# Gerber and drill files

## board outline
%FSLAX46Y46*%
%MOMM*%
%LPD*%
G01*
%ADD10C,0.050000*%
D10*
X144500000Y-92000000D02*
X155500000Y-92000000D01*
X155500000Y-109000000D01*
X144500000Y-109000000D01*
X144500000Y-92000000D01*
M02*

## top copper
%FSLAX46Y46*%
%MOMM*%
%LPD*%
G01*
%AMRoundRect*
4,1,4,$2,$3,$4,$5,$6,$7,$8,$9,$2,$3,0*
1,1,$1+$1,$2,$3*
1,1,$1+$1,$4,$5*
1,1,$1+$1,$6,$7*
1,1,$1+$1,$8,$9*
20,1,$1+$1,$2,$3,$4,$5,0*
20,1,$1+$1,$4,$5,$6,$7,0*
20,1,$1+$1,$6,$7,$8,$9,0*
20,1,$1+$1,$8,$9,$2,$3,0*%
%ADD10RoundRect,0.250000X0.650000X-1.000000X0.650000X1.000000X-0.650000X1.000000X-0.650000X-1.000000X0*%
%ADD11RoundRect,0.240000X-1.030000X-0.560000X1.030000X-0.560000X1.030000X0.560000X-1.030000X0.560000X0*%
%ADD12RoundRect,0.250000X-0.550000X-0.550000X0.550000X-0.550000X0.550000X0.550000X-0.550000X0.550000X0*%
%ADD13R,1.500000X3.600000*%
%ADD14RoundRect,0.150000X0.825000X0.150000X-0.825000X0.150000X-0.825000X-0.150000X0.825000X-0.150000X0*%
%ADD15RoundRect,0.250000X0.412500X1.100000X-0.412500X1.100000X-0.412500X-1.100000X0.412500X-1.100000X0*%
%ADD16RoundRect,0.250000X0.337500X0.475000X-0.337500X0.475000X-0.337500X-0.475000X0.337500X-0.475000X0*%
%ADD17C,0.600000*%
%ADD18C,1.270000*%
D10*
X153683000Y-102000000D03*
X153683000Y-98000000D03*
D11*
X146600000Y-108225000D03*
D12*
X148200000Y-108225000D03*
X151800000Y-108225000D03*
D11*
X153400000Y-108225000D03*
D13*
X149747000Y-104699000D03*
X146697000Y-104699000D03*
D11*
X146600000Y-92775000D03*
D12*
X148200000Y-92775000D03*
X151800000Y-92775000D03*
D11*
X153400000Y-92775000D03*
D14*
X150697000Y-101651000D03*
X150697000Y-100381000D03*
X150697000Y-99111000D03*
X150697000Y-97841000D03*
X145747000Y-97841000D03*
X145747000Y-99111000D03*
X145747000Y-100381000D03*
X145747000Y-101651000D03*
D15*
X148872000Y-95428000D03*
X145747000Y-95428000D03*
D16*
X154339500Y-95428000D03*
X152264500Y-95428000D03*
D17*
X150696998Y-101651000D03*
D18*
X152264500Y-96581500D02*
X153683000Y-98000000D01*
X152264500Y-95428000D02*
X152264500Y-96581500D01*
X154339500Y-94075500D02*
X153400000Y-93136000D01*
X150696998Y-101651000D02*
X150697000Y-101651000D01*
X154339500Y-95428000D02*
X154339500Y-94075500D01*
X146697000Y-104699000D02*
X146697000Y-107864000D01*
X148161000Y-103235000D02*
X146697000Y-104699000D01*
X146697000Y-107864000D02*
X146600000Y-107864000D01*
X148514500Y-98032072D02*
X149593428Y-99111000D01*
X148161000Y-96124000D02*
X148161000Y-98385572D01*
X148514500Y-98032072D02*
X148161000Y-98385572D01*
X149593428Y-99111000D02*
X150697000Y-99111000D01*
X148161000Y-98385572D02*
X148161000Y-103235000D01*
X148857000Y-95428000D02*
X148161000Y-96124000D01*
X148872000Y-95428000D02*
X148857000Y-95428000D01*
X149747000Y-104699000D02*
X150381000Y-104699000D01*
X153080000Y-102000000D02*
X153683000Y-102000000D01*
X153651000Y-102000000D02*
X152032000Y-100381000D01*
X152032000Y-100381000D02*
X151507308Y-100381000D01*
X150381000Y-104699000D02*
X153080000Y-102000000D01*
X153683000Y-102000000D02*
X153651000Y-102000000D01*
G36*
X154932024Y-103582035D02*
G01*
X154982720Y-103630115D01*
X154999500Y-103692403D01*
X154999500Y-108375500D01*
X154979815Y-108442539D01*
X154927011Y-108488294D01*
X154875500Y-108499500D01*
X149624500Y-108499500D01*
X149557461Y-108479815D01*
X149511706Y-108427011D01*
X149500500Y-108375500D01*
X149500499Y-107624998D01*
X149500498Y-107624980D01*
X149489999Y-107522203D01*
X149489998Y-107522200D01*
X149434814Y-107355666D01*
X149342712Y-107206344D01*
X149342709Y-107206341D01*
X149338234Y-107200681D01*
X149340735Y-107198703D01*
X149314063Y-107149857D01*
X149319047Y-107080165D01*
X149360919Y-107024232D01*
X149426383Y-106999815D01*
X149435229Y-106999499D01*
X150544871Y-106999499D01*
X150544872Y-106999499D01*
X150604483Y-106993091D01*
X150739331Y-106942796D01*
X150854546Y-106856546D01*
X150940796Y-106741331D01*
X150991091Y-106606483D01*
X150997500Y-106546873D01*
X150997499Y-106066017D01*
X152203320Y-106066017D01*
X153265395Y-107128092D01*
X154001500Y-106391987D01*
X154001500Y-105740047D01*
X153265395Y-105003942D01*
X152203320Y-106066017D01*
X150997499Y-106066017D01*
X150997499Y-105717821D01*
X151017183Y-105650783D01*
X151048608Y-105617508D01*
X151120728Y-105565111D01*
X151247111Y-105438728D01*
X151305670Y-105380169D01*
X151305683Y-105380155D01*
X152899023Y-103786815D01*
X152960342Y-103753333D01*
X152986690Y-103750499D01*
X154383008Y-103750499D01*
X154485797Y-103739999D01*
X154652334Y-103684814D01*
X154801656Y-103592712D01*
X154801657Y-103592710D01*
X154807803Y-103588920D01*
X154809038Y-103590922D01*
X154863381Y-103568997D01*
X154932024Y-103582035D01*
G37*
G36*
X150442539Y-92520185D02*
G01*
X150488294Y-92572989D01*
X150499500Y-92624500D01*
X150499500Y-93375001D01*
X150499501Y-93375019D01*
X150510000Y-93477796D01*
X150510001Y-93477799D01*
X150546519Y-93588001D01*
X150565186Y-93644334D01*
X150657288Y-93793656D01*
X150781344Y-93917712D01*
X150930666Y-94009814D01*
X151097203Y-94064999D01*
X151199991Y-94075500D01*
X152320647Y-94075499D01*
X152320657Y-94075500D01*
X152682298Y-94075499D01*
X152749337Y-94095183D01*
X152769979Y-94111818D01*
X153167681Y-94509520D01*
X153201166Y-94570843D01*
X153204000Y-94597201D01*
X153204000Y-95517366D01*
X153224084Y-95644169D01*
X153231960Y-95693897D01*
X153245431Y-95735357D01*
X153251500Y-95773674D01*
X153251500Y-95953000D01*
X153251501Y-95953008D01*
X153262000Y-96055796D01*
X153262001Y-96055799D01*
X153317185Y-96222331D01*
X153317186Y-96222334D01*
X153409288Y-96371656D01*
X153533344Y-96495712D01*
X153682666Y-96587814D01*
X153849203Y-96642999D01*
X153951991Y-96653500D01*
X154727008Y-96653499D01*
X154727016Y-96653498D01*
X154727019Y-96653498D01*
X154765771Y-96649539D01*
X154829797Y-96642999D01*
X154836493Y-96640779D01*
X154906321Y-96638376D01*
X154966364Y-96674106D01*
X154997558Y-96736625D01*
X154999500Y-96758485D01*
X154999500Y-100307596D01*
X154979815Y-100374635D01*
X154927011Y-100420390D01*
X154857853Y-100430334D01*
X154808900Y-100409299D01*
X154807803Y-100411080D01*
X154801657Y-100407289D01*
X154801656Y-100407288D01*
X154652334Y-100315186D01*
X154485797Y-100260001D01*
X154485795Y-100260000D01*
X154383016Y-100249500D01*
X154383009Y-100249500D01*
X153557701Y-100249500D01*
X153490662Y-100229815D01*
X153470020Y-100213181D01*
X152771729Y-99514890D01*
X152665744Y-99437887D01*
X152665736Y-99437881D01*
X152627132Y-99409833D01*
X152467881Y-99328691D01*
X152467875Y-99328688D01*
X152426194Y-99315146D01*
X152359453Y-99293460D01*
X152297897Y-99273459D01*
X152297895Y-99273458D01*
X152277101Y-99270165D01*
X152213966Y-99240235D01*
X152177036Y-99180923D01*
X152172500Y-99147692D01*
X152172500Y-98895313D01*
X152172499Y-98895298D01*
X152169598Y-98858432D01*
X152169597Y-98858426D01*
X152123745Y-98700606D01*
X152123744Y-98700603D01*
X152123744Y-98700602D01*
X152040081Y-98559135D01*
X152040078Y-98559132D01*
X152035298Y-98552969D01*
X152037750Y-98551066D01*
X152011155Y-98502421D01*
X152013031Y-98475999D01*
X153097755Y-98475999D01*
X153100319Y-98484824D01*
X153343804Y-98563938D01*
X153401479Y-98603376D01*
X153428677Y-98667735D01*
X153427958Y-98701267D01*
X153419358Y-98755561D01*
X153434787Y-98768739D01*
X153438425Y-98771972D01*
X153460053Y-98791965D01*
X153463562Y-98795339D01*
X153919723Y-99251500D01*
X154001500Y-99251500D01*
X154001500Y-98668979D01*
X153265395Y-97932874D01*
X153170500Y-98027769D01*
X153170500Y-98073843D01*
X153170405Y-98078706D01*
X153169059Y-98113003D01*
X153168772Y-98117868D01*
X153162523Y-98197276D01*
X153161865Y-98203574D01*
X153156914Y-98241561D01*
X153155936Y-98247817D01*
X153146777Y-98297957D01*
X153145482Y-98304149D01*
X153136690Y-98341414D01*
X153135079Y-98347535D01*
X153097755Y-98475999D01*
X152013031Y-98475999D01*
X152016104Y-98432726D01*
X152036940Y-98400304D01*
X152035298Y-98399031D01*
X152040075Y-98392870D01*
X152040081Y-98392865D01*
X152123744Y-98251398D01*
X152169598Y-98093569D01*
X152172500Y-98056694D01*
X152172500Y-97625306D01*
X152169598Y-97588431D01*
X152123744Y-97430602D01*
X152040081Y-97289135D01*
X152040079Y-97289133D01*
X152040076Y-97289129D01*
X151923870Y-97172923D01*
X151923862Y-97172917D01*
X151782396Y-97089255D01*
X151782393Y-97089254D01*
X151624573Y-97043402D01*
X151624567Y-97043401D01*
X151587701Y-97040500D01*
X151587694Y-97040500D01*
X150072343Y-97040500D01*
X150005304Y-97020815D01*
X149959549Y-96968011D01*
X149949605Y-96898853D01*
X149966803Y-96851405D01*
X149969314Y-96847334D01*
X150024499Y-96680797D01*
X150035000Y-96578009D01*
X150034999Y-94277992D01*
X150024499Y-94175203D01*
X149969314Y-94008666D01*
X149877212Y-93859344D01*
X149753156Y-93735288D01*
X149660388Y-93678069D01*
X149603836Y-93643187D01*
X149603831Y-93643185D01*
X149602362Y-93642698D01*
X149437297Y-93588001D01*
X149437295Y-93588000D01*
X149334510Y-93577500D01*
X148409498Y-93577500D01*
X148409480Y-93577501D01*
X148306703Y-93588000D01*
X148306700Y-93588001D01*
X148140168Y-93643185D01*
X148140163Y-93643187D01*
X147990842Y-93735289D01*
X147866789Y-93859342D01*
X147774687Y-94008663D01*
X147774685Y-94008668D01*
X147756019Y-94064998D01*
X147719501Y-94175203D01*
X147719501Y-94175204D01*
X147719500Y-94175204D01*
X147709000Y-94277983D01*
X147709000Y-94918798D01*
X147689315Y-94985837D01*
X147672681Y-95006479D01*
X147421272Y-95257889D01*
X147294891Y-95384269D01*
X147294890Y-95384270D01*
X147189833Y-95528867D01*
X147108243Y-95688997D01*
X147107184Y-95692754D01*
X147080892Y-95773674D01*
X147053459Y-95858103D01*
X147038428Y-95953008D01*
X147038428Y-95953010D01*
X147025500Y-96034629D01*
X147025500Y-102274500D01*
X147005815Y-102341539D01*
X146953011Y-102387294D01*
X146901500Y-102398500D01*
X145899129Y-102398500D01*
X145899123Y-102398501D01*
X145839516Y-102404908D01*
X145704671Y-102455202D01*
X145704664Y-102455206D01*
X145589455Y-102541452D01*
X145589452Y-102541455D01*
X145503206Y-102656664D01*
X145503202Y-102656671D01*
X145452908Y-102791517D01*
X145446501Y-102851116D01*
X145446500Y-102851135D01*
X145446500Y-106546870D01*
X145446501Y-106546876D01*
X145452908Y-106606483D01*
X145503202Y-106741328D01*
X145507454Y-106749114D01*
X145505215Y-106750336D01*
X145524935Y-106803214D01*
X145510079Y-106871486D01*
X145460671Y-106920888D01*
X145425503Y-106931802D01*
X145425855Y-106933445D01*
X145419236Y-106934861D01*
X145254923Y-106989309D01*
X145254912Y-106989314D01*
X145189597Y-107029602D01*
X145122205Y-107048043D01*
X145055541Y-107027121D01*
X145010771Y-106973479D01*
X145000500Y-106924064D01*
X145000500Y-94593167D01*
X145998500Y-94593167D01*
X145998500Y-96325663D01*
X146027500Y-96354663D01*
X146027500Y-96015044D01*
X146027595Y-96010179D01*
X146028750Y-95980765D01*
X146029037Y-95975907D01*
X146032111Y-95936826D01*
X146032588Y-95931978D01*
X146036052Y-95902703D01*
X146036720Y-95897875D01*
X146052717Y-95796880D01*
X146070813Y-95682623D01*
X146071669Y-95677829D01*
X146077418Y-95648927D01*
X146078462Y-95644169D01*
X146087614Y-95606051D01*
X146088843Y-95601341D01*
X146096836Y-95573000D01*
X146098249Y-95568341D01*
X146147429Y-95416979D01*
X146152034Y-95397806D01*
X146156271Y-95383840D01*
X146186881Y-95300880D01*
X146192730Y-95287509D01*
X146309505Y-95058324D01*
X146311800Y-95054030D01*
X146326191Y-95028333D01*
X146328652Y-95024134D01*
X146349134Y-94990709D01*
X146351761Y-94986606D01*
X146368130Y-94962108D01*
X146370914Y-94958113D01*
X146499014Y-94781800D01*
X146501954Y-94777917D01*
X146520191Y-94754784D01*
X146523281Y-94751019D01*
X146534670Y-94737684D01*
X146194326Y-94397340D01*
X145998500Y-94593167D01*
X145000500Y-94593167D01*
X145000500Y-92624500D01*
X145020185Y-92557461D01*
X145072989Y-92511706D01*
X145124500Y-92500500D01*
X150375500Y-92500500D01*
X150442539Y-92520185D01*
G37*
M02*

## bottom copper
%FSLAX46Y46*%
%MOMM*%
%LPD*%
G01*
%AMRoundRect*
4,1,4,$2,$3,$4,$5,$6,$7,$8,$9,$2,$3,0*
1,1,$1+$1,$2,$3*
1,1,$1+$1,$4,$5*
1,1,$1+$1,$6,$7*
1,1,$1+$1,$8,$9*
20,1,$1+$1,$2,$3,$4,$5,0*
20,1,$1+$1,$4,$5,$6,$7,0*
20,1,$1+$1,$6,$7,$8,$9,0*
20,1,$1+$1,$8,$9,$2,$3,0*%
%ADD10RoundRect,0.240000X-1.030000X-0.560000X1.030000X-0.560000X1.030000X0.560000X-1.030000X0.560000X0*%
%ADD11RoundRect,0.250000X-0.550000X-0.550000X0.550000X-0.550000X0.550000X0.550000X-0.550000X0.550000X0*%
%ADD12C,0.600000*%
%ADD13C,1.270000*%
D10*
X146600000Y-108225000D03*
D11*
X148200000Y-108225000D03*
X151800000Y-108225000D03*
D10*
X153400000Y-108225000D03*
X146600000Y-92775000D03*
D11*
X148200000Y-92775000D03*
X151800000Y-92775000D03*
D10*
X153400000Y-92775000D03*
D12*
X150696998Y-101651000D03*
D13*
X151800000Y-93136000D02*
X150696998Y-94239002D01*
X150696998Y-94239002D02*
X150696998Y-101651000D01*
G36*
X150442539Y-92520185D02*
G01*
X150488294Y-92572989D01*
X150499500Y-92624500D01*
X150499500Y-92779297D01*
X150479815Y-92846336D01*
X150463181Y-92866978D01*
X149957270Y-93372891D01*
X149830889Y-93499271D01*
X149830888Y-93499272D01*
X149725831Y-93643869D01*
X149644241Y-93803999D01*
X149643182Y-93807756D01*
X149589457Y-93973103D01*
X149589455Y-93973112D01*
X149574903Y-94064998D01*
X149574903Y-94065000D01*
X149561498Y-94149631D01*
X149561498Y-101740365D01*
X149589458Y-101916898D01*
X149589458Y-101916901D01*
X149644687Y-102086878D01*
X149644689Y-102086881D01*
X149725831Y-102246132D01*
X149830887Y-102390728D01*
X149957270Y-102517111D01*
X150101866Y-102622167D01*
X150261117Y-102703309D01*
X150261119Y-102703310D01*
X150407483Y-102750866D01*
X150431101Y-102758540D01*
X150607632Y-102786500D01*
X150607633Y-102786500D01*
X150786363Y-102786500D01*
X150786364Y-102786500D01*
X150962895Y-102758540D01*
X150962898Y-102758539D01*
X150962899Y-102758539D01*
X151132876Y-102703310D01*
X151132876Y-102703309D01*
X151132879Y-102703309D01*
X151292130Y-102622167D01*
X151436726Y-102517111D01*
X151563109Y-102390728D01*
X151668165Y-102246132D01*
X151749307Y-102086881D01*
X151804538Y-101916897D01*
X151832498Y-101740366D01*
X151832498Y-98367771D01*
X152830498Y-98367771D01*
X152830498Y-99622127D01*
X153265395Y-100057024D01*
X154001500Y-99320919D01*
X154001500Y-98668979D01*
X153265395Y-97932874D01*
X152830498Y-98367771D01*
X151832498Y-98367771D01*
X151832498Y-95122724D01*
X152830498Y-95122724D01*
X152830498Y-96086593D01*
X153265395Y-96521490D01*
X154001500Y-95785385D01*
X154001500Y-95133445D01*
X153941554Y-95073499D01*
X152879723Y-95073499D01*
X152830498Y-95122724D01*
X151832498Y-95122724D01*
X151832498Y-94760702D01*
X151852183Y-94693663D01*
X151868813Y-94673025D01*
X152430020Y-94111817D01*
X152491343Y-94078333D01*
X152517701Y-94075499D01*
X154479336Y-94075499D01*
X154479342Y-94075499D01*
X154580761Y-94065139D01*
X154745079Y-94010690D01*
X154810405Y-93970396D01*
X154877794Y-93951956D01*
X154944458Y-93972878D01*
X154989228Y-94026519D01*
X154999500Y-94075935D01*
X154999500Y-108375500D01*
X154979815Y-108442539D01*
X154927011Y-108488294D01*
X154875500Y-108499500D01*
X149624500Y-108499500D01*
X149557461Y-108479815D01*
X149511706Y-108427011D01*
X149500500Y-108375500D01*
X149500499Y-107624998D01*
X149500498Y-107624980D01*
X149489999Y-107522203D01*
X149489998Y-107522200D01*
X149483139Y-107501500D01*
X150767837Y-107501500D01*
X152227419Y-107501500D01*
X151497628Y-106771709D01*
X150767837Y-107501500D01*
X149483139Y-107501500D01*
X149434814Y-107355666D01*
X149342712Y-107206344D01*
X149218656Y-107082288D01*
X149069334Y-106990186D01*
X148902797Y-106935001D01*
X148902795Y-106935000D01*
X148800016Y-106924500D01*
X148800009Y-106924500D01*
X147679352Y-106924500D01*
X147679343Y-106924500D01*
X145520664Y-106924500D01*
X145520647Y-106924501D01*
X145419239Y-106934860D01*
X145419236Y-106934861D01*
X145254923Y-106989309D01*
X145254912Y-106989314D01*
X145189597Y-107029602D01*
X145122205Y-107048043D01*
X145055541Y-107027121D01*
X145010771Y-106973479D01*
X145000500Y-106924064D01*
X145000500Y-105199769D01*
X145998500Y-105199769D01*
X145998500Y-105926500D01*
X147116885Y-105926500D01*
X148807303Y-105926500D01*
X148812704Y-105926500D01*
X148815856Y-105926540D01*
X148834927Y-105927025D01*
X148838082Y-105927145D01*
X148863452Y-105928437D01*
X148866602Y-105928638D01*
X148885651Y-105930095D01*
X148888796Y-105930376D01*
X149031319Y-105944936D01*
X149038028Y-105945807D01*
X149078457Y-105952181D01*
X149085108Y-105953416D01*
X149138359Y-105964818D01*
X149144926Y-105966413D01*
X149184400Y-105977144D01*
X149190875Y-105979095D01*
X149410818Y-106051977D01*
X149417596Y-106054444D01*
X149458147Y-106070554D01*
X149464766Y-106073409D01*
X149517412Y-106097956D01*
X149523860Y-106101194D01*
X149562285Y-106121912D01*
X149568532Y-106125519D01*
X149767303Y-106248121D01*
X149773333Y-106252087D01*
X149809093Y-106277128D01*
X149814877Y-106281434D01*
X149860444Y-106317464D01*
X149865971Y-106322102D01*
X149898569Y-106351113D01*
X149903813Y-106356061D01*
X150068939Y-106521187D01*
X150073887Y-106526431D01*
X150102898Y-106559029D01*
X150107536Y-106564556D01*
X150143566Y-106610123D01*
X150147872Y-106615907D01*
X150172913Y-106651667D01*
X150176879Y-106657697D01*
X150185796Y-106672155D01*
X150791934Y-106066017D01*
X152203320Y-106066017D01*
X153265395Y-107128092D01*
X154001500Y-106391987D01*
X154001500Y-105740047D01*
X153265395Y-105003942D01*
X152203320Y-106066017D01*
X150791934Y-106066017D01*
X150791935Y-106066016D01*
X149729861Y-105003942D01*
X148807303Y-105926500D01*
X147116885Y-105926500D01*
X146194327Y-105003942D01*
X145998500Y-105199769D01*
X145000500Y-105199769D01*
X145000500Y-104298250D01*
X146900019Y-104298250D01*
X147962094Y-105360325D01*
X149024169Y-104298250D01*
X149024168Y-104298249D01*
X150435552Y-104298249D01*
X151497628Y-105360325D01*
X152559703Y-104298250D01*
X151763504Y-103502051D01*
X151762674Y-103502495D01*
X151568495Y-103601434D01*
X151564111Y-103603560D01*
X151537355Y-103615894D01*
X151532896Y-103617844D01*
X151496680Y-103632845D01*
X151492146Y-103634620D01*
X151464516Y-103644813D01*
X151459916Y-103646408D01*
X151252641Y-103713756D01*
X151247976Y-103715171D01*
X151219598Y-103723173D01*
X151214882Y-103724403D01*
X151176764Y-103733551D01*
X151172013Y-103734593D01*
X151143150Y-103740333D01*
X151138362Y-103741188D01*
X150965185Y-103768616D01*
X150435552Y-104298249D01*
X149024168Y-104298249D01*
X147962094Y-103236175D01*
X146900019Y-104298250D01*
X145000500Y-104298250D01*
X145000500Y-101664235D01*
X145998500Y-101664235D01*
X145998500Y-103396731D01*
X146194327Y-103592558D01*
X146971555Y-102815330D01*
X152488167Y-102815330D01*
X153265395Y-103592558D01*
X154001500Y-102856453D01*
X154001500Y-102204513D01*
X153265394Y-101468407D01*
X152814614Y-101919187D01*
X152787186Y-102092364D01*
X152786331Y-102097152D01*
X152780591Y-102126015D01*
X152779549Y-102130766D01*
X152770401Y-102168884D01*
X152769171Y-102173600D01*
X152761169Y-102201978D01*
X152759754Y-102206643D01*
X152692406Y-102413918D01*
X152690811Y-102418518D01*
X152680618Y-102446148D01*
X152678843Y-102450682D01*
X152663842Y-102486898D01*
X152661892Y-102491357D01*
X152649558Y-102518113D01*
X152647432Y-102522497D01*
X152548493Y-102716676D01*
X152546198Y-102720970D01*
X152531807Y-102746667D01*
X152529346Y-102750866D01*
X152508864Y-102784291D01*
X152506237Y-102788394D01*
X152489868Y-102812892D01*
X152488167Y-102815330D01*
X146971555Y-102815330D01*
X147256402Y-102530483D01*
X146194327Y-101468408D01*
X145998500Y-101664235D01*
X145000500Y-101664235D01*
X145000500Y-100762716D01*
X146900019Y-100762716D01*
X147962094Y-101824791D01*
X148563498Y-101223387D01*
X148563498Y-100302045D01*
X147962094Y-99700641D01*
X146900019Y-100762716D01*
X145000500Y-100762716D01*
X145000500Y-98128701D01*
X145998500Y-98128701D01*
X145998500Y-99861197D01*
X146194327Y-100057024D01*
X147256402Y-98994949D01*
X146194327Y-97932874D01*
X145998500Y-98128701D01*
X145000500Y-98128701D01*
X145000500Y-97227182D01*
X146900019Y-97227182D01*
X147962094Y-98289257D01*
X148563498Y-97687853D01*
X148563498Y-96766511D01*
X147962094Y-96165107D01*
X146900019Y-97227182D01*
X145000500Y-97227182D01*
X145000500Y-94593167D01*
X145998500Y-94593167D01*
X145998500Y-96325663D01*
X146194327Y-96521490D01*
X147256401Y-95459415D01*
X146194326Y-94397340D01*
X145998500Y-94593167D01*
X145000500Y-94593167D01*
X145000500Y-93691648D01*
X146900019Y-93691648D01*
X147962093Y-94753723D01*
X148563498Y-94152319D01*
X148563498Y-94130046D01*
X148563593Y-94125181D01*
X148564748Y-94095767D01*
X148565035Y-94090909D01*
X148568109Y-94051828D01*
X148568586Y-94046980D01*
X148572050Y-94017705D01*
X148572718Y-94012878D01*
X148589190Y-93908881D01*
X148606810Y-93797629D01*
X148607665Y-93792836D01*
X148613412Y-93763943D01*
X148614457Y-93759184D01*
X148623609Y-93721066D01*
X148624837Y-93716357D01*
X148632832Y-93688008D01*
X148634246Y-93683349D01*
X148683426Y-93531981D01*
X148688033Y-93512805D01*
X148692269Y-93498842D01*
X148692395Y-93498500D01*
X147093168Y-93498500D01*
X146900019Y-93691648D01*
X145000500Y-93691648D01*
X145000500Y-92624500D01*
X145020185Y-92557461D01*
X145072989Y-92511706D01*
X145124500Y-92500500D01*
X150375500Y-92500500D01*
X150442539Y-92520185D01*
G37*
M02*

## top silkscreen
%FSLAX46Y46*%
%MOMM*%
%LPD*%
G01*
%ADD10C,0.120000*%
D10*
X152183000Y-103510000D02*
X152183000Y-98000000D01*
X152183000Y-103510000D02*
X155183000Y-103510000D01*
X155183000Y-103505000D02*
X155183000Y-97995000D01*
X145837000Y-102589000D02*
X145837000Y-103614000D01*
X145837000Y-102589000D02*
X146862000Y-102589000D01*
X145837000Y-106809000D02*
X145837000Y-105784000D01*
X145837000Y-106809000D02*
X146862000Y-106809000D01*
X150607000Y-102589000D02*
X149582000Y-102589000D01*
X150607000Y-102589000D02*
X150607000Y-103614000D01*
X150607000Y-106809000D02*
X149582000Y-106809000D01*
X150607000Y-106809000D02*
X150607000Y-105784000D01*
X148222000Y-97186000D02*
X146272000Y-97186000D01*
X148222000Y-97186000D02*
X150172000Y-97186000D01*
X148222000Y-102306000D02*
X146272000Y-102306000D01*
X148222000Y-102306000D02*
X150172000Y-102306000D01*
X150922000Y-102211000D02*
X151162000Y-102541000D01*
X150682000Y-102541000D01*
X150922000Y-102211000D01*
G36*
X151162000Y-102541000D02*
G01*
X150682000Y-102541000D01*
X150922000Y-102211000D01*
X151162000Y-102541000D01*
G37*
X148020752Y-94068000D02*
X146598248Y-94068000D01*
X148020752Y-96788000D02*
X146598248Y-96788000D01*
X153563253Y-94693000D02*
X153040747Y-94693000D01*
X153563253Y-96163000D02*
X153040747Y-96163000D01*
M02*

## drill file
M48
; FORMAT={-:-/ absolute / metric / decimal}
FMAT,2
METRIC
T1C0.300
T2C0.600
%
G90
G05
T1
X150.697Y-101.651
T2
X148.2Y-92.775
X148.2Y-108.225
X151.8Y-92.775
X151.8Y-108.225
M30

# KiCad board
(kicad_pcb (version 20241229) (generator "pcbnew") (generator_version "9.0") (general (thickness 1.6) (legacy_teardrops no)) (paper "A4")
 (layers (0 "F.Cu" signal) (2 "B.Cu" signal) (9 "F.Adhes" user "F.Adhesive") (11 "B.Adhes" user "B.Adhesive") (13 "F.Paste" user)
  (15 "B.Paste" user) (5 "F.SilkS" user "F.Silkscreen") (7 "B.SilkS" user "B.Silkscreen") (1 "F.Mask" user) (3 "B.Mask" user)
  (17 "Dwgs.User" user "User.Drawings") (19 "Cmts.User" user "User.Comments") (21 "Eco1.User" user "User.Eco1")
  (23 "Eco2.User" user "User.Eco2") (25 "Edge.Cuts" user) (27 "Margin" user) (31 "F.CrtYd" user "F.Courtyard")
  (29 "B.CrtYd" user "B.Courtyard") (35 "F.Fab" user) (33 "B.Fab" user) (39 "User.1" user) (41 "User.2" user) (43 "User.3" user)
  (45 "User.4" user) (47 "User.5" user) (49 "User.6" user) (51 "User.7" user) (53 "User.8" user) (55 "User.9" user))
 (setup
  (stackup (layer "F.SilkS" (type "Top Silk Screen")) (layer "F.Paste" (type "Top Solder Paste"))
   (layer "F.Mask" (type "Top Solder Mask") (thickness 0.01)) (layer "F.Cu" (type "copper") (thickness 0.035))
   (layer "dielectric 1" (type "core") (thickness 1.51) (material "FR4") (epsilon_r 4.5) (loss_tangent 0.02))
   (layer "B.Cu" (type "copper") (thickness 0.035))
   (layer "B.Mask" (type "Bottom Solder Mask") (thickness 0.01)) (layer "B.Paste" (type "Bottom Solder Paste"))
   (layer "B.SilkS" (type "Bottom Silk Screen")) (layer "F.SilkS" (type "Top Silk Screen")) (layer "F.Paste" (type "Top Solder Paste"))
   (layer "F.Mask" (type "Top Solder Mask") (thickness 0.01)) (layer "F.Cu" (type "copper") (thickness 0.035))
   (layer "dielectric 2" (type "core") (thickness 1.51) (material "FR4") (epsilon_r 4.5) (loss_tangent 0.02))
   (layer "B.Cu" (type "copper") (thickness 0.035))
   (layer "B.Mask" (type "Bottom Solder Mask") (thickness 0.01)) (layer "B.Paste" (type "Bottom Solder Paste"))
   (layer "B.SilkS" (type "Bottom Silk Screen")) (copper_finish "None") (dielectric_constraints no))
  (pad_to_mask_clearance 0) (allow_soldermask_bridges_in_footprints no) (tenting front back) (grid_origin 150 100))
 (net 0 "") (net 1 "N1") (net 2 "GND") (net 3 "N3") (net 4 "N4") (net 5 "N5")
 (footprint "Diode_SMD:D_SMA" (layer "F.Cu") (at 153.683 100 90)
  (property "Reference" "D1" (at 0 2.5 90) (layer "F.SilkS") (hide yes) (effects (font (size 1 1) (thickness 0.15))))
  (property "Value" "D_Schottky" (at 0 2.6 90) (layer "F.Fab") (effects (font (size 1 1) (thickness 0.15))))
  (fp_line (start -3.51 -1.5) (end 2 -1.5) (stroke (width 0.12) (type solid)) (layer "F.SilkS"))
  (fp_line (start -3.51 -1.5) (end -3.51 1.5) (stroke (width 0.12) (type solid)) (layer "F.SilkS"))
  (fp_line (start -3.505 1.5) (end 2.005 1.5) (stroke (width 0.12) (type solid)) (layer "F.SilkS"))
  (pad "1" smd roundrect (at -2 0 90) (size 2.5 1.8) (layers "F.Cu" "F.Mask" "F.Paste") (roundrect_rratio 0.1388888889) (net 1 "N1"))
  (pad "2" smd roundrect (at 2 0 90) (size 2.5 1.8) (layers "F.Cu" "F.Mask" "F.Paste") (roundrect_rratio 0.1388888889) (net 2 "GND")))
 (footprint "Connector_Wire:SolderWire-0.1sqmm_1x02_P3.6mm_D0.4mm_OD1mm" (layer "F.Cu") (at 148.2 108.225)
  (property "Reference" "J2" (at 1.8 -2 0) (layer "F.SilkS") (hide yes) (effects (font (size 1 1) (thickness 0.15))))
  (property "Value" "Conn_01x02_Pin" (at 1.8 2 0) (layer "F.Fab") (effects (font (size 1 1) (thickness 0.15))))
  (pad "1" connect roundrect (at -1.6 0) (size 2.54 1.6) (layers "F.Cu" "F.Mask") (roundrect_rratio 0.15) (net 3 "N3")
   (thermal_bridge_angle 45))
  (pad "1" connect roundrect (at -1.6 0) (size 2.54 1.6) (layers "B.Cu" "B.Mask") (roundrect_rratio 0.15) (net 3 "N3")
   (thermal_bridge_angle 45))
  (pad "1" thru_hole roundrect (at 0 0) (size 1.6 1.6) (drill 0.6) (layers "*.Cu" "*.Mask") (remove_unused_layers no)
   (roundrect_rratio 0.15625) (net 3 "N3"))
  (pad "2" thru_hole roundrect (at 3.6 0) (size 1.6 1.6) (drill 0.6) (layers "*.Cu" "*.Mask") (remove_unused_layers no)
   (roundrect_rratio 0.15625) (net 2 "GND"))
  (pad "2" connect roundrect (at 5.2 0) (size 2.54 1.6) (layers "F.Cu" "F.Mask") (roundrect_rratio 0.15) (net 2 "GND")
   (thermal_bridge_angle 45))
  (pad "2" connect roundrect (at 5.2 0) (size 2.54 1.6) (layers "B.Cu" "B.Mask") (roundrect_rratio 0.15) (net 2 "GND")
   (thermal_bridge_angle 45)))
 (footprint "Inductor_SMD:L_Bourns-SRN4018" (layer "F.Cu") (at 148.222 104.699 180)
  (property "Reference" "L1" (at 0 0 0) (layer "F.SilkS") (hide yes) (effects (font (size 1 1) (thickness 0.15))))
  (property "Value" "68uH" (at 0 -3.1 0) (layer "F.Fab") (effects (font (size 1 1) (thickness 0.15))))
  (fp_line (start 2.385 2.11) (end 2.385 1.085) (stroke (width 0.12) (type solid)) (layer "F.SilkS"))
  (fp_line (start 2.385 2.11) (end 1.36 2.11) (stroke (width 0.12) (type solid)) (layer "F.SilkS"))
  (fp_line (start 2.385 -2.11) (end 2.385 -1.085) (stroke (width 0.12) (type solid)) (layer "F.SilkS"))
  (fp_line (start 2.385 -2.11) (end 1.36 -2.11) (stroke (width 0.12) (type solid)) (layer "F.SilkS"))
  (fp_line (start -2.385 2.11) (end -1.36 2.11) (stroke (width 0.12) (type solid)) (layer "F.SilkS"))
  (fp_line (start -2.385 2.11) (end -2.385 1.085) (stroke (width 0.12) (type solid)) (layer "F.SilkS"))
  (fp_line (start -2.385 -2.11) (end -1.36 -2.11) (stroke (width 0.12) (type solid)) (layer "F.SilkS"))
  (fp_line (start -2.385 -2.11) (end -2.385 -1.085) (stroke (width 0.12) (type solid)) (layer "F.SilkS"))
  (pad "1" smd rect (at -1.525 0 180) (size 1.5 3.6) (layers "F.Cu" "F.Mask" "F.Paste") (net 1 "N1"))
  (pad "2" smd rect (at 1.525 0 180) (size 1.5 3.6) (layers "F.Cu" "F.Mask" "F.Paste") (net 3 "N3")))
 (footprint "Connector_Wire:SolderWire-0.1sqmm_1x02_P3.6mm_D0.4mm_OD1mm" (layer "F.Cu") (at 148.2 92.775)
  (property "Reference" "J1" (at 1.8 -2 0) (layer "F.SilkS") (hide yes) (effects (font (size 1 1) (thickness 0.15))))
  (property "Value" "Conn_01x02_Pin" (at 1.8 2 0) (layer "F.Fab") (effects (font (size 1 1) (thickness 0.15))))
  (pad "1" connect roundrect (at -1.6 0) (size 2.54 1.6) (layers "F.Cu" "F.Mask") (roundrect_rratio 0.15) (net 2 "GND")
   (thermal_bridge_angle 45))
  (pad "1" connect roundrect (at -1.6 0) (size 2.54 1.6) (layers "B.Cu" "B.Mask") (roundrect_rratio 0.15) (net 2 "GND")
   (thermal_bridge_angle 45))
  (pad "1" thru_hole roundrect (at 0 0) (size 1.6 1.6) (drill 0.6) (layers "*.Cu" "*.Mask") (remove_unused_layers no)
   (roundrect_rratio 0.15625) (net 2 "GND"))
  (pad "2" thru_hole roundrect (at 3.6 0) (size 1.6 1.6) (drill 0.6) (layers "*.Cu" "*.Mask") (remove_unused_layers no)
   (roundrect_rratio 0.15625) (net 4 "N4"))
  (pad "2" connect roundrect (at 5.2 0) (size 2.54 1.6) (layers "F.Cu" "F.Mask") (roundrect_rratio 0.15) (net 4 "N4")
   (thermal_bridge_angle 45))
  (pad "2" connect roundrect (at 5.2 0) (size 2.54 1.6) (layers "B.Cu" "B.Mask") (roundrect_rratio 0.15) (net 4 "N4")
   (thermal_bridge_angle 45)))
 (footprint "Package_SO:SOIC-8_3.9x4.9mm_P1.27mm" (layer "F.Cu") (at 148.222 99.746 180)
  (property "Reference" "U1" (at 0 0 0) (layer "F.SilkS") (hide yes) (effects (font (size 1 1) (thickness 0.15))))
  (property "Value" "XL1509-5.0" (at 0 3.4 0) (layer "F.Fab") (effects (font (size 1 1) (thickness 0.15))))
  (fp_line (start 0 2.56) (end 1.95 2.56) (stroke (width 0.12) (type solid)) (layer "F.SilkS"))
  (fp_line (start 0 2.56) (end -1.95 2.56) (stroke (width 0.12) (type solid)) (layer "F.SilkS"))
  (fp_line (start 0 -2.56) (end 1.95 -2.56) (stroke (width 0.12) (type solid)) (layer "F.SilkS"))
  (fp_line (start 0 -2.56) (end -1.95 -2.56) (stroke (width 0.12) (type solid)) (layer "F.SilkS"))
  (fp_poly
   (pts (xy -2.7 -2.465) (xy -2.94 -2.795) (xy -2.46 -2.795) (xy -2.7 -2.465)) (stroke (width 0.12) (type solid)) (fill yes)
   (layer "F.SilkS"))
  (pad "1" smd roundrect (at -2.475 -1.905 180) (size 1.95 0.6) (layers "F.Cu" "F.Mask" "F.Paste") (roundrect_rratio 0.25) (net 4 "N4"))
  (pad "2" smd roundrect (at -2.475 -0.635 180) (size 1.95 0.6) (layers "F.Cu" "F.Mask" "F.Paste") (roundrect_rratio 0.25) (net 1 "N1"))
  (pad "3" smd roundrect (at -2.475 0.635 180) (size 1.95 0.6) (layers "F.Cu" "F.Mask" "F.Paste") (roundrect_rratio 0.25) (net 3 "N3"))
  (pad "4" smd roundrect (at -2.475 1.905 180) (size 1.95 0.6) (layers "F.Cu" "F.Mask" "F.Paste") (roundrect_rratio 0.25) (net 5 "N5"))
  (pad "5" smd roundrect (at 2.475 1.905 180) (size 1.95 0.6) (layers "F.Cu" "F.Mask" "F.Paste") (roundrect_rratio 0.25) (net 2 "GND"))
  (pad "6" smd roundrect (at 2.475 0.635 180) (size 1.95 0.6) (layers "F.Cu" "F.Mask" "F.Paste") (roundrect_rratio 0.25) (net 2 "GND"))
  (pad "7" smd roundrect (at 2.475 -0.635 180) (size 1.95 0.6) (layers "F.Cu" "F.Mask" "F.Paste") (roundrect_rratio 0.25) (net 2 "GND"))
  (pad "8" smd roundrect (at 2.475 -1.905 180) (size 1.95 0.6) (layers "F.Cu" "F.Mask" "F.Paste") (roundrect_rratio 0.25) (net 2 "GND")))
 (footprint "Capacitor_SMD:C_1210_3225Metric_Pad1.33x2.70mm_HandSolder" (layer "F.Cu") (at 147.3095 95.428 180)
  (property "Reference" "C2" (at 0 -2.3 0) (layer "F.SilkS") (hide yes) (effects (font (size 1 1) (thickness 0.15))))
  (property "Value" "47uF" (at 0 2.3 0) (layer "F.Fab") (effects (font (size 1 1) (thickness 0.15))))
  (fp_line (start -0.711252 1.36) (end 0.711252 1.36) (stroke (width 0.12) (type solid)) (layer "F.SilkS"))
  (fp_line (start -0.711252 -1.36) (end 0.711252 -1.36) (stroke (width 0.12) (type solid)) (layer "F.SilkS"))
  (pad "1" smd roundrect (at -1.5625 0 180) (size 1.325 2.7) (layers "F.Cu" "F.Mask" "F.Paste") (roundrect_rratio 0.188679) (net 3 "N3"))
  (pad "2" smd roundrect (at 1.5625 0 180) (size 1.325 2.7) (layers "F.Cu" "F.Mask" "F.Paste") (roundrect_rratio 0.188679) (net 2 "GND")))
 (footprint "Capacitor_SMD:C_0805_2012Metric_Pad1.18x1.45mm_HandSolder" (layer "F.Cu") (at 153.302 95.428 180)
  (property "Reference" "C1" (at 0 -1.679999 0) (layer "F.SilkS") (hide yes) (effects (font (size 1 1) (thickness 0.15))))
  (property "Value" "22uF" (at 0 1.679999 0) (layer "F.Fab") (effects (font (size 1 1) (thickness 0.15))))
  (fp_line (start -0.261253 0.735) (end 0.261253 0.735) (stroke (width 0.12) (type solid)) (layer "F.SilkS"))
  (fp_line (start -0.261253 -0.735) (end 0.261253 -0.735) (stroke (width 0.12) (type solid)) (layer "F.SilkS"))
  (pad "1" smd roundrect (at -1.0375 0 180) (size 1.175 1.45) (layers "F.Cu" "F.Mask" "F.Paste") (roundrect_rratio 0.212766) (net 4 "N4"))
  (pad "2" smd roundrect (at 1.0375 0 180) (size 1.175 1.45) (layers "F.Cu" "F.Mask" "F.Paste") (roundrect_rratio 0.212766) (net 2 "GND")))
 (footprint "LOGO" (layer "B.Cu") (at 150 100 180)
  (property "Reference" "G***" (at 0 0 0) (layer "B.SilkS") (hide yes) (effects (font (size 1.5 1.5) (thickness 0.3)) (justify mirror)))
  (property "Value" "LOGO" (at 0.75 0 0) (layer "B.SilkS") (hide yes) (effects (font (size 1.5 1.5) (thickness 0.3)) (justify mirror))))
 (gr_rect (start 144.5 92) (end 155.5 109) (stroke (width 0.05) (type default)) (fill no) (layer "Edge.Cuts"))
 (segment (start 152.2645 96.5815) (end 153.683 98) (width 1.27) (layer "F.Cu") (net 2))
 (segment (start 152.2645 95.428) (end 152.2645 96.5815) (width 1.27) (layer "F.Cu") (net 2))
 (segment (start 154.3395 94.0755) (end 153.4 93.136) (width 1.27) (layer "F.Cu") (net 4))
 (segment (start 150.696998 101.651) (end 150.697 101.651) (width 1.27) (layer "F.Cu") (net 4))
 (segment (start 154.3395 95.428) (end 154.3395 94.0755) (width 1.27) (layer "F.Cu") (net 4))
 (via (at 150.696998 101.651) (size 0.6) (drill 0.3) (layers "F.Cu" "B.Cu") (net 4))
 (segment (start 151.8 93.136) (end 150.696998 94.239002) (width 1.27) (layer "B.Cu") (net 4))
 (segment (start 150.696998 94.239002) (end 150.696998 101.651) (width 1.27) (layer "B.Cu") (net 4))
 (segment (start 146.697 104.699) (end 146.697 107.864) (width 1.27) (layer "F.Cu") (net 3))
 (segment (start 148.161 103.235) (end 146.697 104.699) (width 1.27) (layer "F.Cu") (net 3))
 (segment (start 146.697 107.864) (end 146.6 107.864) (width 1.27) (layer "F.Cu") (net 3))
 (segment (start 148.5145 98.032072) (end 149.593428 99.111) (width 1.27) (layer "F.Cu") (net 3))
 (segment (start 148.161 96.124) (end 148.161 98.385572) (width 1.27) (layer "F.Cu") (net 3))
 (segment (start 148.5145 98.032072) (end 148.161 98.385572) (width 1.27) (layer "F.Cu") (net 3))
 (segment (start 149.593428 99.111) (end 150.697 99.111) (width 1.27) (layer "F.Cu") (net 3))
 (segment (start 148.161 98.385572) (end 148.161 103.235) (width 1.27) (layer "F.Cu") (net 3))
 (segment (start 148.857 95.428) (end 148.161 96.124) (width 1.27) (layer "F.Cu") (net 3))
 (segment (start 148.872 95.428) (end 148.857 95.428) (width 1.27) (layer "F.Cu") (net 3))
 (segment (start 149.747 104.699) (end 150.381 104.699) (width 1.27) (layer "F.Cu") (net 1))
 (segment (start 153.08 102) (end 153.683 102) (width 1.27) (layer "F.Cu") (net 1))
 (segment (start 153.651 102) (end 152.032 100.381) (width 1.27) (layer "F.Cu") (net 1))
 (segment (start 152.032 100.381) (end 151.507308 100.381) (width 1.27) (layer "F.Cu") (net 1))
 (segment (start 150.381 104.699) (end 153.08 102) (width 1.27) (layer "F.Cu") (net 1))
 (segment (start 153.683 102) (end 153.651 102) (width 1.27) (layer "F.Cu") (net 1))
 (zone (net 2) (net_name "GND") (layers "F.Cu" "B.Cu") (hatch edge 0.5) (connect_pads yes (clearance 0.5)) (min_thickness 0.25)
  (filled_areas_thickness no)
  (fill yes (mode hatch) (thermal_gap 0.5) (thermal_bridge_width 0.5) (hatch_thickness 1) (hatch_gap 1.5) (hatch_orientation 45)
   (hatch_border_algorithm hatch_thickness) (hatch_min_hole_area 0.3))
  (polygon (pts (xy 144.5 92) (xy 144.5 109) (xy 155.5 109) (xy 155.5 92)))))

